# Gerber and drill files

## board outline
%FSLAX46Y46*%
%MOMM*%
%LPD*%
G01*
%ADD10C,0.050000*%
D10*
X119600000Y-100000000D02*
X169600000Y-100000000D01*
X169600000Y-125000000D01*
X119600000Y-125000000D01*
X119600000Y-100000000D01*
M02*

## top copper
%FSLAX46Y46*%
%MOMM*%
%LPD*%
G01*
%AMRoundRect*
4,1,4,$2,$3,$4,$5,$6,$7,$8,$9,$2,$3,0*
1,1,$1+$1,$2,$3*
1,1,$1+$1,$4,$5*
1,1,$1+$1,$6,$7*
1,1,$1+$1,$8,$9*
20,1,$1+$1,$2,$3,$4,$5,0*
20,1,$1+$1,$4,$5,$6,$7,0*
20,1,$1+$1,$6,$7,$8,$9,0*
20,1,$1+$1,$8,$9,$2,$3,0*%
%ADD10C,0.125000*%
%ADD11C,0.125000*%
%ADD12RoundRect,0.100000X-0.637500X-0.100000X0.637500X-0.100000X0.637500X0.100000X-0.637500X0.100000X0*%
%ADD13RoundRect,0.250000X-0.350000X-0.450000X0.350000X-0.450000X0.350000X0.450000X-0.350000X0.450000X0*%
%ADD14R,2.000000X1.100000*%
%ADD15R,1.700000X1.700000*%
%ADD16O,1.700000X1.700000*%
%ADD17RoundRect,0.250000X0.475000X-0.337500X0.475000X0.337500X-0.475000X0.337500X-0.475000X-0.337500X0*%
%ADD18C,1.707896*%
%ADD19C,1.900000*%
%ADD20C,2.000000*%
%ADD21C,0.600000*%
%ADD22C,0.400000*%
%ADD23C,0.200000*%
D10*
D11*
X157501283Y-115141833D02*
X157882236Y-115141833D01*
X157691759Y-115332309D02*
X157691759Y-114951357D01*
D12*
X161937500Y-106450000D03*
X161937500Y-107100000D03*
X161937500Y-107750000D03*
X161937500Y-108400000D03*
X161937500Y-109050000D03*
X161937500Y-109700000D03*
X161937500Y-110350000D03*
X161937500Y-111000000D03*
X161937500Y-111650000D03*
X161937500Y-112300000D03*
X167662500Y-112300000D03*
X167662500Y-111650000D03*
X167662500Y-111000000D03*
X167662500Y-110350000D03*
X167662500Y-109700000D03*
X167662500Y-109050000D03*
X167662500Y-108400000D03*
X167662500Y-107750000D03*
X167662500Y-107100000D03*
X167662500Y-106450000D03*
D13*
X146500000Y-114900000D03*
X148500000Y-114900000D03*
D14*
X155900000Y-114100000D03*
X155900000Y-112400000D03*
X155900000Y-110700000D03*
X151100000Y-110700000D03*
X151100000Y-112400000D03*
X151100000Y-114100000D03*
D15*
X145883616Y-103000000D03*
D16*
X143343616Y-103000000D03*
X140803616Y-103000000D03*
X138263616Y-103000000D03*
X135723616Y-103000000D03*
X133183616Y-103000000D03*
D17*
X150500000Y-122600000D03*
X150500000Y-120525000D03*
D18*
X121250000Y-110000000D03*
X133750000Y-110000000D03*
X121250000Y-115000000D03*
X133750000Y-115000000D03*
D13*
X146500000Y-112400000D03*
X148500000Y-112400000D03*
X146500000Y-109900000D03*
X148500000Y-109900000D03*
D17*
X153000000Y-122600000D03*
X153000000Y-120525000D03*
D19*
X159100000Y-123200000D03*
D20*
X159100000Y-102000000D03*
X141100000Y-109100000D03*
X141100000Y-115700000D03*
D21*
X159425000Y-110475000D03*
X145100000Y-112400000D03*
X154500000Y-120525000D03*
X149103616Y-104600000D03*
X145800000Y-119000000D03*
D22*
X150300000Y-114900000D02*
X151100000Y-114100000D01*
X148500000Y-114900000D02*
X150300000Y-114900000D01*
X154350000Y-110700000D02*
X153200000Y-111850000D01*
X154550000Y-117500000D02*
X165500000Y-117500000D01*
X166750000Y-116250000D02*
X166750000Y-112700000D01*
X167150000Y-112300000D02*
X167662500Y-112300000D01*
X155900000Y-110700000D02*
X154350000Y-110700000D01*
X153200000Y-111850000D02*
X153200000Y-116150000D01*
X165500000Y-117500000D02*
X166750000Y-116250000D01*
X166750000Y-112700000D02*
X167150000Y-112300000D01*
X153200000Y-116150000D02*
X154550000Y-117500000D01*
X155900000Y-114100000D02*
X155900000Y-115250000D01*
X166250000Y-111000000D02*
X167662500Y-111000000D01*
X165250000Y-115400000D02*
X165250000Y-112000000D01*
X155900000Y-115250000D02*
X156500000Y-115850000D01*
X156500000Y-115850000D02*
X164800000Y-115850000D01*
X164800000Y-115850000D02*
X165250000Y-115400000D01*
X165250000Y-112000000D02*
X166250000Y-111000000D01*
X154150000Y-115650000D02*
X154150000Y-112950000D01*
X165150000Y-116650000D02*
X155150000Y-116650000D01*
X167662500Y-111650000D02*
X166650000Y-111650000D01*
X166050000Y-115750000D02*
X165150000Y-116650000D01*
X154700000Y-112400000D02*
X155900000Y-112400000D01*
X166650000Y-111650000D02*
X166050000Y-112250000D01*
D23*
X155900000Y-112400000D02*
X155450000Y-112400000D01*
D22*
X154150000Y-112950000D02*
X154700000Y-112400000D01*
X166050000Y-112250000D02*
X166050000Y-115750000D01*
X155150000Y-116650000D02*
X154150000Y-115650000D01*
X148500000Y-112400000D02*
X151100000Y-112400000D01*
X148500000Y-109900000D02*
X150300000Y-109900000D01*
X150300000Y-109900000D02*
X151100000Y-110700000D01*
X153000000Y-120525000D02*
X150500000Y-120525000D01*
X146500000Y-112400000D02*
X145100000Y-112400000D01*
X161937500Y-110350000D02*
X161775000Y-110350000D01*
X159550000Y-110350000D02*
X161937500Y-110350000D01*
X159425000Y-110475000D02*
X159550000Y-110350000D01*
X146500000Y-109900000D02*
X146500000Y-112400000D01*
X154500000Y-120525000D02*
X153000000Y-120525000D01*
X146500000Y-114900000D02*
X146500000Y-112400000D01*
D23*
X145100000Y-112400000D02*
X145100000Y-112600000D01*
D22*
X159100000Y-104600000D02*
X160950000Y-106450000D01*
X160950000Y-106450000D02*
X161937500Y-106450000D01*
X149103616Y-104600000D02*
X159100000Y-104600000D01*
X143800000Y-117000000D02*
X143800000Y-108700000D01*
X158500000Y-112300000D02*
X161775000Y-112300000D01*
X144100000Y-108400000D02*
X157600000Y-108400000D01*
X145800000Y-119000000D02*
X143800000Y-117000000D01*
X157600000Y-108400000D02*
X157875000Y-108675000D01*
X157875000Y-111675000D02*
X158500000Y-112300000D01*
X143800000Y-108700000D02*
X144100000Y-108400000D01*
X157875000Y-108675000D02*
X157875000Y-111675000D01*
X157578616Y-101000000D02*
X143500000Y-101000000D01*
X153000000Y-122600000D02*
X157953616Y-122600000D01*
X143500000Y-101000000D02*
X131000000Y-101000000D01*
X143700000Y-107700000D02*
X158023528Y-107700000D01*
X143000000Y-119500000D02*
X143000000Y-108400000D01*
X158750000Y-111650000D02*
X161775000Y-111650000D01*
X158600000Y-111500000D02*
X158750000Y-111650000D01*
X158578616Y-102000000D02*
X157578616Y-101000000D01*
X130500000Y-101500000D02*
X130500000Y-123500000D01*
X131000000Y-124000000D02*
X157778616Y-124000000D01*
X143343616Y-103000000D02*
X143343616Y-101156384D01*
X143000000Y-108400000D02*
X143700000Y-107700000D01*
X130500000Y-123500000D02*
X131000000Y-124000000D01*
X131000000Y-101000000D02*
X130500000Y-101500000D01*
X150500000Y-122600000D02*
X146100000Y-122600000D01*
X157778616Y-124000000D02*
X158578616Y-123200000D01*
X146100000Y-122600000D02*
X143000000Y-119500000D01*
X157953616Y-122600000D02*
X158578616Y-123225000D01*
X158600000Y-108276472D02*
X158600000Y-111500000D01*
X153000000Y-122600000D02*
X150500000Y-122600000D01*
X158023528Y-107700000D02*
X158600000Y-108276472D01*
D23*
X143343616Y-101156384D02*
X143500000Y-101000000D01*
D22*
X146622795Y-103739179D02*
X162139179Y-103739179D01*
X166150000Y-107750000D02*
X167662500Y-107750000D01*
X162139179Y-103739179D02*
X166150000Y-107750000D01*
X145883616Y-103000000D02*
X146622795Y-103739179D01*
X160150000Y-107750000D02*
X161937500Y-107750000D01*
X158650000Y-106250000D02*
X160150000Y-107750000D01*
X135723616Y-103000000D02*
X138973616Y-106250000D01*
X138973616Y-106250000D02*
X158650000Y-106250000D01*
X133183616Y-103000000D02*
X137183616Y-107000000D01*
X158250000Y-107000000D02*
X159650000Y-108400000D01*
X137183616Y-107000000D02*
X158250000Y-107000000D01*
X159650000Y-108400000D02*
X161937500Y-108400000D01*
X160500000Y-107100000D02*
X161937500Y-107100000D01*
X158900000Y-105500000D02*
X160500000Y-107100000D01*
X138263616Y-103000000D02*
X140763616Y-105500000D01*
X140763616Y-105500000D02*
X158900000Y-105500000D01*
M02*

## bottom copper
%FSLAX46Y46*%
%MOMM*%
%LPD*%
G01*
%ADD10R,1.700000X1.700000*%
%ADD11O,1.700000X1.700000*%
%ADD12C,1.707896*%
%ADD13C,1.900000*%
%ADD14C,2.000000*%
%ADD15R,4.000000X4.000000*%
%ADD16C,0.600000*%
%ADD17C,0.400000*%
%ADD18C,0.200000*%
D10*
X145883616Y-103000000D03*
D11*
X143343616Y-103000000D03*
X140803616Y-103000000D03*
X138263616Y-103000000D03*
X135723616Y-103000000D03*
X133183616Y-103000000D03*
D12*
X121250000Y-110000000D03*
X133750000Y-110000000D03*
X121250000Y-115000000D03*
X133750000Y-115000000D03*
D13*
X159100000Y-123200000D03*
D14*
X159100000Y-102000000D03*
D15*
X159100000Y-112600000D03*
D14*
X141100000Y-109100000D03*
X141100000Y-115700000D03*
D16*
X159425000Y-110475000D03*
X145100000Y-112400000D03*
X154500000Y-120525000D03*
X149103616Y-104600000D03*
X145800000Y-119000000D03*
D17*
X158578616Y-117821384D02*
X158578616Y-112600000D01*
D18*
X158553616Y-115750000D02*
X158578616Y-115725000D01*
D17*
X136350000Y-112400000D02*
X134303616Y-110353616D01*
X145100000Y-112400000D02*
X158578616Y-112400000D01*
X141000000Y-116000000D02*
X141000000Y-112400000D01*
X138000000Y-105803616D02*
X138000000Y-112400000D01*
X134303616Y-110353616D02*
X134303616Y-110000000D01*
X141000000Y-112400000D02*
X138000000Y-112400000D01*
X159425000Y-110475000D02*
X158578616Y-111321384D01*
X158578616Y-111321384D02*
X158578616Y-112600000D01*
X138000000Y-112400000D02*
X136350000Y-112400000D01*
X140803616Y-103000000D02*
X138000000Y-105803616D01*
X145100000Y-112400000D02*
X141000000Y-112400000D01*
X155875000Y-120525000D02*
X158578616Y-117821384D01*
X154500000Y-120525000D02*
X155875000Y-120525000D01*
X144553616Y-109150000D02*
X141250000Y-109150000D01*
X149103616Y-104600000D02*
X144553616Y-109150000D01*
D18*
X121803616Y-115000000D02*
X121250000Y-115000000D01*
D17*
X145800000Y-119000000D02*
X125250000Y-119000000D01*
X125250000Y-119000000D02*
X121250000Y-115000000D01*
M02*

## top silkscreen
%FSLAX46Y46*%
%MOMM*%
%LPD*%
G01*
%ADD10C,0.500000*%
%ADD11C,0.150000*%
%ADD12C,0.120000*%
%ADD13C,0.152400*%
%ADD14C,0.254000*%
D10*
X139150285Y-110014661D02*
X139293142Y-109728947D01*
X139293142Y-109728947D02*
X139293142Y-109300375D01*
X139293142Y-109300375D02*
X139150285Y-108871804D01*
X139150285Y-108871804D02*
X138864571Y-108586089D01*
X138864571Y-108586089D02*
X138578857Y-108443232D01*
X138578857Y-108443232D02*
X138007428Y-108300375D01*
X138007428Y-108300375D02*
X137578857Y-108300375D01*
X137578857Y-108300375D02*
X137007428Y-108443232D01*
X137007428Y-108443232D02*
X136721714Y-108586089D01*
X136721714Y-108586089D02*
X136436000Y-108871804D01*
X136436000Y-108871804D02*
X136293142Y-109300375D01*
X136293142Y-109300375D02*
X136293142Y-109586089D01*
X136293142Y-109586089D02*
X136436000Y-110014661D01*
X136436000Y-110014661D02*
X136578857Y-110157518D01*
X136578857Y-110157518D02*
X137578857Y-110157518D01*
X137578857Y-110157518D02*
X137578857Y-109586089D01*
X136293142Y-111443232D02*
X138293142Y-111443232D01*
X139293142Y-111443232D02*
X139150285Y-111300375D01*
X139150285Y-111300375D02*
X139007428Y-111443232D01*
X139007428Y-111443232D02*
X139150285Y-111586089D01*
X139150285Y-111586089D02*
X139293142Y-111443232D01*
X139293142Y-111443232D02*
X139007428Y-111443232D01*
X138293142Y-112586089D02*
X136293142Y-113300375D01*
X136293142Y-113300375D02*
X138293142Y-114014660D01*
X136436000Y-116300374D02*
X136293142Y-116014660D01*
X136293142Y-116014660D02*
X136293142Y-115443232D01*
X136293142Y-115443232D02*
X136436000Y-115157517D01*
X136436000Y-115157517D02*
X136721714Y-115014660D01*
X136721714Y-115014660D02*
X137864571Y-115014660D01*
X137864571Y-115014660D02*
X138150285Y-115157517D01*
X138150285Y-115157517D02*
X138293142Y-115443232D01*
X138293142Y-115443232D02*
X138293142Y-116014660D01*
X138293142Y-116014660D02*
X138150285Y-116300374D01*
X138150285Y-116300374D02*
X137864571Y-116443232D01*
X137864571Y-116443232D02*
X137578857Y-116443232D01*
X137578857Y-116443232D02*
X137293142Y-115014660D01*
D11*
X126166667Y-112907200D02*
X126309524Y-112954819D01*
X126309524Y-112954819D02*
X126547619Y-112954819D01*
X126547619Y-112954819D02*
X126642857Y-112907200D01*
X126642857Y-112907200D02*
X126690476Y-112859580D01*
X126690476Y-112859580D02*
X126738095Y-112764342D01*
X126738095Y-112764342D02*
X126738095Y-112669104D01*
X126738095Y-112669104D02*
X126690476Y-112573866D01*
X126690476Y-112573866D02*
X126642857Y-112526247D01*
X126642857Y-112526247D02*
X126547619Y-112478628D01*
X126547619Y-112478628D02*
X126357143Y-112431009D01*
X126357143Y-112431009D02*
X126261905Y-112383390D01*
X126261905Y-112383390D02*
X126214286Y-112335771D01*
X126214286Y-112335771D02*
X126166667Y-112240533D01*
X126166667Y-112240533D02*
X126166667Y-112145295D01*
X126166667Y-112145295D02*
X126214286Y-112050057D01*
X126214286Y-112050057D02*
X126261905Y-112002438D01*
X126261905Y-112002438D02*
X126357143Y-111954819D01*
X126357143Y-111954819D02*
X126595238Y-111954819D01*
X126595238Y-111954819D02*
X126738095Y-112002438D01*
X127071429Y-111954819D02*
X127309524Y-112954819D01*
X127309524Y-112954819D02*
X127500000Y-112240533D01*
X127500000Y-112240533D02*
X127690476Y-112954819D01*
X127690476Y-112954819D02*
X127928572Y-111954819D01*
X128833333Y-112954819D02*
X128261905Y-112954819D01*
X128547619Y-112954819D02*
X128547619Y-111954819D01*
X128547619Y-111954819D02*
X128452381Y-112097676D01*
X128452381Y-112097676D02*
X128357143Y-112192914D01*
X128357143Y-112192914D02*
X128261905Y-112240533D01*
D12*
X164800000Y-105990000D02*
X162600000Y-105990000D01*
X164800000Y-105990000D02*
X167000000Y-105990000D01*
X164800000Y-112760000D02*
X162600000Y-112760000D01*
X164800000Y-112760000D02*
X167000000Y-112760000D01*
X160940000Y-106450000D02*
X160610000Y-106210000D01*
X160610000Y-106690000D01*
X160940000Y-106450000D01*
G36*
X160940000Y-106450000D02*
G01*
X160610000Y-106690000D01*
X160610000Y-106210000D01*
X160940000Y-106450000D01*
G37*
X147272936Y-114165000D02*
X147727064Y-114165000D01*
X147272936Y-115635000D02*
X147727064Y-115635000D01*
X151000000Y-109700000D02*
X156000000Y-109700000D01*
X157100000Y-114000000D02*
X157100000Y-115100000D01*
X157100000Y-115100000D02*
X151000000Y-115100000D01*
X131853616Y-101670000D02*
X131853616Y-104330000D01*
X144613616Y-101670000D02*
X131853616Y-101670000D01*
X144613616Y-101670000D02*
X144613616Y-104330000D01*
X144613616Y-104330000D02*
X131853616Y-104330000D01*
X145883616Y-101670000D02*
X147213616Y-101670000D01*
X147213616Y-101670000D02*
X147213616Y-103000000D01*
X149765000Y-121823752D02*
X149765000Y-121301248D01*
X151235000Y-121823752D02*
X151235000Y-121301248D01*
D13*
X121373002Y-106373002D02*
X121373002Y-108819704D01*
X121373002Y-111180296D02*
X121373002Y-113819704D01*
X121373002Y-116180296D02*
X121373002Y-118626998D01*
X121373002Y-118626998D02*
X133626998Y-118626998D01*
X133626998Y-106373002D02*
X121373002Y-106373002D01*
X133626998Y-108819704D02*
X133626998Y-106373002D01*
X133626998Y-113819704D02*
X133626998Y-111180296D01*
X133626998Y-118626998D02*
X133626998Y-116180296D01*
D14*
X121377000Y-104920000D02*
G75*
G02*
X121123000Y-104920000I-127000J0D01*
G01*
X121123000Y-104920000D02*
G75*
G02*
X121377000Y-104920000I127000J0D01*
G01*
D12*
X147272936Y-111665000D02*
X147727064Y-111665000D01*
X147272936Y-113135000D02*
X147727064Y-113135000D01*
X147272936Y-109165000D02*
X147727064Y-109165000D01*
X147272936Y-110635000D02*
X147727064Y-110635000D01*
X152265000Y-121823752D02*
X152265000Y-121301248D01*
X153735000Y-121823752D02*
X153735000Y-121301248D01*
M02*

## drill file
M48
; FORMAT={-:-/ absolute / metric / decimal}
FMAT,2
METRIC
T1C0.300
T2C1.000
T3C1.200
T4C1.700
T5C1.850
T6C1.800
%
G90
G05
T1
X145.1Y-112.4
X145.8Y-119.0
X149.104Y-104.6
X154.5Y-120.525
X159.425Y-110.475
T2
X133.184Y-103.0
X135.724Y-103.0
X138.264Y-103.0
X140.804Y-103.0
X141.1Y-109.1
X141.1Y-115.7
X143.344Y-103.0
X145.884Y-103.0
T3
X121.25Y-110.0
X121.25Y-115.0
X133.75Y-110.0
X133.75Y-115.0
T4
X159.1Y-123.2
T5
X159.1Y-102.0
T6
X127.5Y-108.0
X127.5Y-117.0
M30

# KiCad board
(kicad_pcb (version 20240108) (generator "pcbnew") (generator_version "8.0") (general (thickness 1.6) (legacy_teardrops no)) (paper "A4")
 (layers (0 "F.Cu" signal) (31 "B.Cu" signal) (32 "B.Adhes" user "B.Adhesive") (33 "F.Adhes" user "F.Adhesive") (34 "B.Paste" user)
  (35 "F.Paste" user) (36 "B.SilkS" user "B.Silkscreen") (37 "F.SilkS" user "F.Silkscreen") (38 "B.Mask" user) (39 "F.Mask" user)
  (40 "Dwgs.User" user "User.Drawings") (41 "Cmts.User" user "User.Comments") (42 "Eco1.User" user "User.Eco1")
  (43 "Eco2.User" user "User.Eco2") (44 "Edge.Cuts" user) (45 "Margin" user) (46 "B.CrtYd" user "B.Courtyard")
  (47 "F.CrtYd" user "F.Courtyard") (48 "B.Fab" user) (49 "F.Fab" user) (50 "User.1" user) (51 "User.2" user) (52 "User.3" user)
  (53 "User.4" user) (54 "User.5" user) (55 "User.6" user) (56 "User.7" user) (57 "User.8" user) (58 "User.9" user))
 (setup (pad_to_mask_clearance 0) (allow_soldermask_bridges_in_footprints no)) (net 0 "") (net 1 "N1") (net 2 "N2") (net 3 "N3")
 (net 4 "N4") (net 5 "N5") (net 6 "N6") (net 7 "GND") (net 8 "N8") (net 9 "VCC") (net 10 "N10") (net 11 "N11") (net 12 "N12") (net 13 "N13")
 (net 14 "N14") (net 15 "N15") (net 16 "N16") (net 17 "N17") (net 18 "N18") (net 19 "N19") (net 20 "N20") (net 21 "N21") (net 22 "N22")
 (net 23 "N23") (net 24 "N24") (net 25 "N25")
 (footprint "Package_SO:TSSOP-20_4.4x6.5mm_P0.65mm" (layer "F.Cu") (at 164.8 109.375)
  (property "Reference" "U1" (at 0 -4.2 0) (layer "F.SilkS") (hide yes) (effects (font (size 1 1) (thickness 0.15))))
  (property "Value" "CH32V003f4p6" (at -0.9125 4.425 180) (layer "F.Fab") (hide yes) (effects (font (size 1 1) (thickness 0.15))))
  (fp_line (start 0 -3.385) (end -2.2 -3.385) (stroke (width 0.12) (type solid)) (layer "F.SilkS"))
  (fp_line (start 0 -3.385) (end 2.2 -3.385) (stroke (width 0.12) (type solid)) (layer "F.SilkS"))
  (fp_line (start 0 3.385) (end -2.2 3.385) (stroke (width 0.12) (type solid)) (layer "F.SilkS"))
  (fp_line (start 0 3.385) (end 2.2 3.385) (stroke (width 0.12) (type solid)) (layer "F.SilkS"))
  (fp_poly
   (pts (xy -3.86 -2.925) (xy -4.19 -3.165) (xy -4.19 -2.685) (xy -3.86 -2.925)) (stroke (width 0.12) (type solid)) (fill solid)
   (layer "F.SilkS"))
  (pad "1" smd roundrect (at -2.8625 -2.925) (size 1.475 0.4) (layers "F.Cu" "F.Paste" "F.Mask") (roundrect_rratio 0.25) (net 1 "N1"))
  (pad "2" smd roundrect (at -2.8625 -2.275) (size 1.475 0.4) (layers "F.Cu" "F.Paste" "F.Mask") (roundrect_rratio 0.25) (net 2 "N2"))
  (pad "3" smd roundrect (at -2.8625 -1.625) (size 1.475 0.4) (layers "F.Cu" "F.Paste" "F.Mask") (roundrect_rratio 0.25) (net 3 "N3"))
  (pad "4" smd roundrect (at -2.8625 -0.975) (size 1.475 0.4) (layers "F.Cu" "F.Paste" "F.Mask") (roundrect_rratio 0.25) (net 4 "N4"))
  (pad "5" smd roundrect (at -2.8625 -0.325) (size 1.475 0.4) (layers "F.Cu" "F.Paste" "F.Mask") (roundrect_rratio 0.25) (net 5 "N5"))
  (pad "6" smd roundrect (at -2.8625 0.325) (size 1.475 0.4) (layers "F.Cu" "F.Paste" "F.Mask") (roundrect_rratio 0.25) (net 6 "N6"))
  (pad "7" smd roundrect (at -2.8625 0.975) (size 1.475 0.4) (layers "F.Cu" "F.Paste" "F.Mask") (roundrect_rratio 0.25) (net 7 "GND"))
  (pad "8" smd roundrect (at -2.8625 1.625) (size 1.475 0.4) (layers "F.Cu" "F.Paste" "F.Mask") (roundrect_rratio 0.25) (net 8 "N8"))
  (pad "9" smd roundrect (at -2.8625 2.275) (size 1.475 0.4) (layers "F.Cu" "F.Paste" "F.Mask") (roundrect_rratio 0.25) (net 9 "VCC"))
  (pad "10" smd roundrect (at -2.8625 2.925) (size 1.475 0.4) (layers "F.Cu" "F.Paste" "F.Mask") (roundrect_rratio 0.25) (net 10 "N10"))
  (pad "11" smd roundrect (at 2.8625 2.925) (size 1.475 0.4) (layers "F.Cu" "F.Paste" "F.Mask") (roundrect_rratio 0.25) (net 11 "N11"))
  (pad "12" smd roundrect (at 2.8625 2.275) (size 1.475 0.4) (layers "F.Cu" "F.Paste" "F.Mask") (roundrect_rratio 0.25) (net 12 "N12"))
  (pad "13" smd roundrect (at 2.8625 1.625) (size 1.475 0.4) (layers "F.Cu" "F.Paste" "F.Mask") (roundrect_rratio 0.25) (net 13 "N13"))
  (pad "14" smd roundrect (at 2.8625 0.975) (size 1.475 0.4) (layers "F.Cu" "F.Paste" "F.Mask") (roundrect_rratio 0.25) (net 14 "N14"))
  (pad "15" smd roundrect (at 2.8625 0.325) (size 1.475 0.4) (layers "F.Cu" "F.Paste" "F.Mask") (roundrect_rratio 0.25) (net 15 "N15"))
  (pad "16" smd roundrect (at 2.8625 -0.325) (size 1.475 0.4) (layers "F.Cu" "F.Paste" "F.Mask") (roundrect_rratio 0.25) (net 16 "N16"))
  (pad "17" smd roundrect (at 2.8625 -0.975) (size 1.475 0.4) (layers "F.Cu" "F.Paste" "F.Mask") (roundrect_rratio 0.25) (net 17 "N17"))
  (pad "18" smd roundrect (at 2.8625 -1.625) (size 1.475 0.4) (layers "F.Cu" "F.Paste" "F.Mask") (roundrect_rratio 0.25) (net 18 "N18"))
  (pad "19" smd roundrect (at 2.8625 -2.275) (size 1.475 0.4) (layers "F.Cu" "F.Paste" "F.Mask") (roundrect_rratio 0.25) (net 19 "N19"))
  (pad "20" smd roundrect (at 2.8625 -2.925) (size 1.475 0.4) (layers "F.Cu" "F.Paste" "F.Mask") (roundrect_rratio 0.25) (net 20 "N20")))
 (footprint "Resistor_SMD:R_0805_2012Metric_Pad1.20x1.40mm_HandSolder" (layer "F.Cu") (at 147.5 114.9)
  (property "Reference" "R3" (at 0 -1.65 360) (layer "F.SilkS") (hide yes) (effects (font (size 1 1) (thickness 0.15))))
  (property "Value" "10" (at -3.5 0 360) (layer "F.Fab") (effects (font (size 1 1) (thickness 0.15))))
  (fp_line (start -0.227064 -0.735) (end 0.227064 -0.735) (stroke (width 0.12) (type solid)) (layer "F.SilkS"))
  (fp_line (start -0.227064 0.735) (end 0.227064 0.735) (stroke (width 0.12) (type solid)) (layer "F.SilkS"))
  (pad "1" smd roundrect (at -1 0) (size 1.2 1.4) (layers "F.Cu" "F.Paste" "F.Mask") (roundrect_rratio 0.208333) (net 7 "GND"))
  (pad "2" smd roundrect (at 1 0) (size 1.2 1.4) (layers "F.Cu" "F.Paste" "F.Mask") (roundrect_rratio 0.208333) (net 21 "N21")))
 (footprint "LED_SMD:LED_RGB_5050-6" (layer "F.Cu") (at 153.5 112.4 180)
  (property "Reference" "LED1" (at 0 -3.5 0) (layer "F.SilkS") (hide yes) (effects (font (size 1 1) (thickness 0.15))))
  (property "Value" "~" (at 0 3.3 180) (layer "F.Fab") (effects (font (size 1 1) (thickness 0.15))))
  (fp_line (start 2.5 2.7) (end -2.5 2.7) (stroke (width 0.12) (type solid)) (layer "F.SilkS"))
  (fp_line (start -3.6 -1.6) (end -3.6 -2.7) (stroke (width 0.12) (type solid)) (layer "F.SilkS"))
  (fp_line (start -3.6 -2.7) (end 2.5 -2.7) (stroke (width 0.12) (type solid)) (layer "F.SilkS"))
  (pad "1" smd rect (at -2.4 -1.7 270) (size 1.1 2) (layers "F.Cu" "F.Paste" "F.Mask") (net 13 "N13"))
  (pad "2" smd rect (at -2.4 0 270) (size 1.1 2) (layers "F.Cu" "F.Paste" "F.Mask") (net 12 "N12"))
  (pad "3" smd rect (at -2.4 1.7 270) (size 1.1 2) (layers "F.Cu" "F.Paste" "F.Mask") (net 11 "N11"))
  (pad "4" smd rect (at 2.4 1.7 270) (size 1.1 2) (layers "F.Cu" "F.Paste" "F.Mask") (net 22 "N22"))
  (pad "5" smd rect (at 2.4 0 270) (size 1.1 2) (layers "F.Cu" "F.Paste" "F.Mask") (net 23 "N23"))
  (pad "6" smd rect (at 2.4 -1.7 270) (size 1.1 2) (layers "F.Cu" "F.Paste" "F.Mask") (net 21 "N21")))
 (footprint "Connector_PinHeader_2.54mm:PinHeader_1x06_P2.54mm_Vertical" (layer "F.Cu") (at 145.883616 103 -90)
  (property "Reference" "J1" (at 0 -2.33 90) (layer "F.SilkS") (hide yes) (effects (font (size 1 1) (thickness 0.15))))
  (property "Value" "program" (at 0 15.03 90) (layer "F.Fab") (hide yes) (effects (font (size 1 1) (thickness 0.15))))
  (fp_line (start -1.33 14.03) (end 1.33 14.03) (stroke (width 0.12) (type solid)) (layer "F.SilkS"))
  (fp_line (start -1.33 1.27) (end -1.33 14.03) (stroke (width 0.12) (type solid)) (layer "F.SilkS"))
  (fp_line (start -1.33 1.27) (end 1.33 1.27) (stroke (width 0.12) (type solid)) (layer "F.SilkS"))
  (fp_line (start 1.33 1.27) (end 1.33 14.03) (stroke (width 0.12) (type solid)) (layer "F.SilkS"))
  (fp_line (start -1.33 0) (end -1.33 -1.33) (stroke (width 0.12) (type solid)) (layer "F.SilkS"))
  (fp_line (start -1.33 -1.33) (end 0 -1.33) (stroke (width 0.12) (type solid)) (layer "F.SilkS"))
  (pad "1" thru_hole rect (at 0 0 270) (size 1.7 1.7) (drill 1) (layers "*.Cu" "*.Mask") (remove_unused_layers no) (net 18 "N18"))
  (pad "2" thru_hole oval (at 0 2.54 270) (size 1.7 1.7) (drill 1) (layers "*.Cu" "*.Mask") (remove_unused_layers no) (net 9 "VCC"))
  (pad "3" thru_hole oval (at 0 5.08 270) (size 1.7 1.7) (drill 1) (layers "*.Cu" "*.Mask") (remove_unused_layers no) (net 7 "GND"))
  (pad "4" thru_hole oval (at 0 7.62 270) (size 1.7 1.7) (drill 1) (layers "*.Cu" "*.Mask") (remove_unused_layers no) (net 2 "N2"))
  (pad "5" thru_hole oval (at 0 10.16 270) (size 1.7 1.7) (drill 1) (layers "*.Cu" "*.Mask") (remove_unused_layers no) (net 3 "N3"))
  (pad "6" thru_hole oval (at 0 12.7 270) (size 1.7 1.7) (drill 1) (layers "*.Cu" "*.Mask") (remove_unused_layers no) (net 4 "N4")))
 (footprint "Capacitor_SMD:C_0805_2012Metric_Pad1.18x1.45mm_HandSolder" (layer "F.Cu") (at 150.5 121.5625 90)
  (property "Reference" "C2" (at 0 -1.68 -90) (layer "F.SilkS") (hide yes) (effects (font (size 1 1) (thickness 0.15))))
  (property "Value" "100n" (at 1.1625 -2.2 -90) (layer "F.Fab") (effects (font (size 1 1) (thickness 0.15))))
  (fp_line (start -0.261252 -0.735) (end 0.261252 -0.735) (stroke (width 0.12) (type solid)) (layer "F.SilkS"))
  (fp_line (start -0.261252 0.735) (end 0.261252 0.735) (stroke (width 0.12) (type solid)) (layer "F.SilkS"))
  (pad "1" smd roundrect (at -1.0375 0 90) (size 1.175 1.45) (layers "F.Cu" "F.Paste" "F.Mask") (roundrect_rratio 0.212766) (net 9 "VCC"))
  (pad "2" smd roundrect (at 1.0375 0 90) (size 1.175 1.45) (layers "F.Cu" "F.Paste" "F.Mask") (roundrect_rratio 0.212766) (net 7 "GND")))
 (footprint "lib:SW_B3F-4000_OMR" (layer "F.Cu") (at 121.25 110)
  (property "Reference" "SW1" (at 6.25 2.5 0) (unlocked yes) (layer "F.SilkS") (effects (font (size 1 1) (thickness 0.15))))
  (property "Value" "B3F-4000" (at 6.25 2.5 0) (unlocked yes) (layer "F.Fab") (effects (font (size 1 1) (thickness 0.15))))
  (fp_line (start 0.123002 -3.626998) (end 0.123002 -1.180296) (stroke (width 0.1524) (type solid)) (layer "F.SilkS"))
  (fp_line (start 0.123002 1.180296) (end 0.123002 3.819704) (stroke (width 0.1524) (type solid)) (layer "F.SilkS"))
  (fp_line (start 0.123002 6.180296) (end 0.123002 8.626998) (stroke (width 0.1524) (type solid)) (layer "F.SilkS"))
  (fp_line (start 0.123002 8.626998) (end 12.376998 8.626998) (stroke (width 0.1524) (type solid)) (layer "F.SilkS"))
  (fp_line (start 12.376998 -3.626998) (end 0.123002 -3.626998) (stroke (width 0.1524) (type solid)) (layer "F.SilkS"))
  (fp_line (start 12.376998 -1.180296) (end 12.376998 -3.626998) (stroke (width 0.1524) (type solid)) (layer "F.SilkS"))
  (fp_line (start 12.376998 3.819704) (end 12.376998 1.180296) (stroke (width 0.1524) (type solid)) (layer "F.SilkS"))
  (fp_line (start 12.376998 8.626998) (end 12.376998 6.180296) (stroke (width 0.1524) (type solid)) (layer "F.SilkS"))
  (fp_circle (center 0 -5.08) (end 0.127 -5.08) (stroke (width 0.254) (type solid)) (fill none) (layer "F.SilkS"))
  (pad "" np_thru_hole circle (at 6.25 -2) (size 1.799996 1.799996) (drill 1.799996) (layers "*.Cu" "*.Mask"))
  (pad "" np_thru_hole circle (at 6.25 7) (size 1.799996 1.799996) (drill 1.799996) (layers "*.Cu" "*.Mask"))
  (pad "1" thru_hole circle (at 0 0) (size 1.707896 1.707896) (drill 1.199896) (layers "*.Cu" "*.Mask") (remove_unused_layers no)
   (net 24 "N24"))
  (pad "2" thru_hole circle (at 12.5 0) (size 1.707896 1.707896) (drill 1.199896) (layers "*.Cu" "*.Mask") (remove_unused_layers no)
   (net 7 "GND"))
  (pad "3" thru_hole circle (at 0 5) (size 1.707896 1.707896) (drill 1.199896) (layers "*.Cu" "*.Mask") (remove_unused_layers no)
   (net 10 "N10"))
  (pad "4" thru_hole circle (at 12.5 5) (size 1.707896 1.707896) (drill 1.199896) (layers "*.Cu" "*.Mask") (remove_unused_layers no)
   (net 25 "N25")))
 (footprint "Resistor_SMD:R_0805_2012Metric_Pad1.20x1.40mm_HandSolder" (layer "F.Cu") (at 147.5 112.4)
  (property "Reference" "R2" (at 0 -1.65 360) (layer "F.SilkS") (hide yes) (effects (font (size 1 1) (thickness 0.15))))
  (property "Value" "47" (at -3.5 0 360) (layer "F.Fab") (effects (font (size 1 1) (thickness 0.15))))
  (fp_line (start -0.227064 -0.735) (end 0.227064 -0.735) (stroke (width 0.12) (type solid)) (layer "F.SilkS"))
  (fp_line (start -0.227064 0.735) (end 0.227064 0.735) (stroke (width 0.12) (type solid)) (layer "F.SilkS"))
  (pad "1" smd roundrect (at -1 0) (size 1.2 1.4) (layers "F.Cu" "F.Paste" "F.Mask") (roundrect_rratio 0.208333) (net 7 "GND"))
  (pad "2" smd roundrect (at 1 0) (size 1.2 1.4) (layers "F.Cu" "F.Paste" "F.Mask") (roundrect_rratio 0.208333) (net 23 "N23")))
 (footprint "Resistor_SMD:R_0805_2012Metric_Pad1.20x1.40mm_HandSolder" (layer "F.Cu") (at 147.5 109.9)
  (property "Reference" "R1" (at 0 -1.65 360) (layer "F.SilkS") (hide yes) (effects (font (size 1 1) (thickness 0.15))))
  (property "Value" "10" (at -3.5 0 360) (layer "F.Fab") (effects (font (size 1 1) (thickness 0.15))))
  (fp_line (start -0.227064 -0.735) (end 0.227064 -0.735) (stroke (width 0.12) (type solid)) (layer "F.SilkS"))
  (fp_line (start -0.227064 0.735) (end 0.227064 0.735) (stroke (width 0.12) (type solid)) (layer "F.SilkS"))
  (pad "1" smd roundrect (at -1 0) (size 1.2 1.4) (layers "F.Cu" "F.Paste" "F.Mask") (roundrect_rratio 0.208333) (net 7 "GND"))
  (pad "2" smd roundrect (at 1 0) (size 1.2 1.4) (layers "F.Cu" "F.Paste" "F.Mask") (roundrect_rratio 0.208333) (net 22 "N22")))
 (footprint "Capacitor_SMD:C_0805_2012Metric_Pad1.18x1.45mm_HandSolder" (layer "F.Cu") (at 153 121.5625 90)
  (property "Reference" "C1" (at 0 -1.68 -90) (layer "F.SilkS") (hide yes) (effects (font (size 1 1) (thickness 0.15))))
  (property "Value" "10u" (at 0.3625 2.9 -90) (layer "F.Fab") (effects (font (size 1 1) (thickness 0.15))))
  (fp_line (start -0.261252 -0.735) (end 0.261252 -0.735) (stroke (width 0.12) (type solid)) (layer "F.SilkS"))
  (fp_line (start -0.261252 0.735) (end 0.261252 0.735) (stroke (width 0.12) (type solid)) (layer "F.SilkS"))
  (pad "1" smd roundrect (at -1.0375 0 90) (size 1.175 1.45) (layers "F.Cu" "F.Paste" "F.Mask") (roundrect_rratio 0.212766) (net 9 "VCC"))
  (pad "2" smd roundrect (at 1.0375 0 90) (size 1.175 1.45) (layers "F.Cu" "F.Paste" "F.Mask") (roundrect_rratio 0.212766) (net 7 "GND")))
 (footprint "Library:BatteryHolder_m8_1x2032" (layer "B.Cu") (at 159.1 112.6 90)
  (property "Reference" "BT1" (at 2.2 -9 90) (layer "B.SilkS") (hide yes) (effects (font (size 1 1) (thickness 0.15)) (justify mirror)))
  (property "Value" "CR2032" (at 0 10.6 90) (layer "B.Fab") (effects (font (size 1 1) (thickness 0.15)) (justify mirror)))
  (pad "1" thru_hole circle (at -10.6 0 90) (size 1.9 1.9) (drill 1.7) (layers "*.Cu" "*.Mask") (remove_unused_layers no) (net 9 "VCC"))
  (pad "1" thru_hole circle (at 10.6 0 90) (size 2 2) (drill 1.85) (layers "*.Cu" "*.Mask") (remove_unused_layers no) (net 9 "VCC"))
  (pad "2" smd rect (at 0 0 90) (size 4 4) (layers "B.Cu" "B.Paste" "B.Mask") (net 7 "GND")))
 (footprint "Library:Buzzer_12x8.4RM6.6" (layer "B.Cu") (at 141.1 109.1 -90)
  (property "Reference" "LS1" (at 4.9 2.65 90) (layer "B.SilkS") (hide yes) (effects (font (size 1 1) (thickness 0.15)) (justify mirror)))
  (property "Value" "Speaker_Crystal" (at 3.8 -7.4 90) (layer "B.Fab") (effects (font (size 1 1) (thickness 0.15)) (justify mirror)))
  (pad "1" thru_hole circle (at 0 0 270) (size 2 2) (drill 1) (layers "*.Cu" "*.Mask") (remove_unused_layers no) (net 1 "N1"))
  (pad "2" thru_hole circle (at 6.6 0 270) (size 2 2) (drill 1) (layers "*.Cu" "*.Mask") (remove_unused_layers no) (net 7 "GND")))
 (gr_rect (start 119.6 100) (end 169.6 125) (stroke (width 0.05) (type default)) (fill none) (layer "Edge.Cuts"))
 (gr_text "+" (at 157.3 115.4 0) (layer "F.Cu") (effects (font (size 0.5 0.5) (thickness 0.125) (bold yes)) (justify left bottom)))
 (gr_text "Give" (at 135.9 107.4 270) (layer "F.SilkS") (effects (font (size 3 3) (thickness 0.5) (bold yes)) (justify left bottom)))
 (segment (start 150.3 114.9) (end 151.1 114.1) (width 0.4) (layer "F.Cu") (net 21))
 (segment (start 148.5 114.9) (end 150.3 114.9) (width 0.4) (layer "F.Cu") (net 21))
 (segment (start 154.35 110.7) (end 153.2 111.85) (width 0.4) (layer "F.Cu") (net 11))
 (segment (start 154.55 117.5) (end 165.5 117.5) (width 0.4) (layer "F.Cu") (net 11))
 (segment (start 166.75 116.25) (end 166.75 112.7) (width 0.4) (layer "F.Cu") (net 11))
 (segment (start 167.15 112.3) (end 167.6625 112.3) (width 0.4) (layer "F.Cu") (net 11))
 (segment (start 155.9 110.7) (end 154.35 110.7) (width 0.4) (layer "F.Cu") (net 11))
 (segment (start 153.2 111.85) (end 153.2 116.15) (width 0.4) (layer "F.Cu") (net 11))
 (segment (start 165.5 117.5) (end 166.75 116.25) (width 0.4) (layer "F.Cu") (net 11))
 (segment (start 166.75 112.7) (end 167.15 112.3) (width 0.4) (layer "F.Cu") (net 11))
 (segment (start 153.2 116.15) (end 154.55 117.5) (width 0.4) (layer "F.Cu") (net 11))
 (segment (start 155.9 114.1) (end 155.9 115.25) (width 0.4) (layer "F.Cu") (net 13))
 (segment (start 166.25 111) (end 167.6625 111) (width 0.4) (layer "F.Cu") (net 13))
 (segment (start 165.25 115.4) (end 165.25 112) (width 0.4) (layer "F.Cu") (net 13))
 (segment (start 155.9 115.25) (end 156.5 115.85) (width 0.4) (layer "F.Cu") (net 13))
 (segment (start 156.5 115.85) (end 164.8 115.85) (width 0.4) (layer "F.Cu") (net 13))
 (segment (start 164.8 115.85) (end 165.25 115.4) (width 0.4) (layer "F.Cu") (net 13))
 (segment (start 165.25 112) (end 166.25 111) (width 0.4) (layer "F.Cu") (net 13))
 (segment (start 154.15 115.65) (end 154.15 112.95) (width 0.4) (layer "F.Cu") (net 12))
 (segment (start 165.15 116.65) (end 155.15 116.65) (width 0.4) (layer "F.Cu") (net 12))
 (segment (start 167.6625 111.65) (end 166.65 111.65) (width 0.4) (layer "F.Cu") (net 12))
 (segment (start 166.05 115.75) (end 165.15 116.65) (width 0.4) (layer "F.Cu") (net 12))
 (segment (start 154.7 112.4) (end 155.9 112.4) (width 0.4) (layer "F.Cu") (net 12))
 (segment (start 166.65 111.65) (end 166.05 112.25) (width 0.4) (layer "F.Cu") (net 12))
 (segment (start 155.9 112.4) (end 155.45 112.4) (width 0.2) (layer "F.Cu") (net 12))
 (segment (start 154.15 112.95) (end 154.7 112.4) (width 0.4) (layer "F.Cu") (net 12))
 (segment (start 166.05 112.25) (end 166.05 115.75) (width 0.4) (layer "F.Cu") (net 12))
 (segment (start 155.15 116.65) (end 154.15 115.65) (width 0.4) (layer "F.Cu") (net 12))
 (segment (start 148.5 112.4) (end 151.1 112.4) (width 0.4) (layer "F.Cu") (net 23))
 (segment (start 148.5 109.9) (end 150.3 109.9) (width 0.4) (layer "F.Cu") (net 22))
 (segment (start 150.3 109.9) (end 151.1 110.7) (width 0.4) (layer "F.Cu") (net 22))
 (segment (start 153 120.525) (end 150.5 120.525) (width 0.4) (layer "F.Cu") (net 7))
 (segment (start 146.5 112.4) (end 145.1 112.4) (width 0.4) (layer "F.Cu") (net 7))
 (segment (start 161.9375 110.35) (end 161.775 110.35) (width 0.4) (layer "F.Cu") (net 7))
 (segment (start 159.55 110.35) (end 161.9375 110.35) (width 0.4) (layer "F.Cu") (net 7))
 (segment (start 159.425 110.475) (end 159.55 110.35) (width 0.4) (layer "F.Cu") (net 7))
 (segment (start 146.5 109.9) (end 146.5 112.4) (width 0.4) (layer "F.Cu") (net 7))
 (segment (start 154.5 120.525) (end 153 120.525) (width 0.4) (layer "F.Cu") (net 7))
 (segment (start 146.5 114.9) (end 146.5 112.4) (width 0.4) (layer "F.Cu") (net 7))
 (segment (start 145.1 112.4) (end 145.1 112.6) (width 0.2) (layer "F.Cu") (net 7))
 (via (at 159.425 110.475) (size 0.6) (drill 0.3) (layers "F.Cu" "B.Cu") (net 7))
 (via (at 145.1 112.4) (size 0.6) (drill 0.3) (layers "F.Cu" "B.Cu") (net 7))
 (via (at 154.5 120.525) (size 0.6) (drill 0.3) (layers "F.Cu" "B.Cu") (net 7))
 (segment (start 158.578616 117.821384) (end 158.578616 112.6) (width 0.4) (layer "B.Cu") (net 7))
 (segment (start 158.553616 115.75) (end 158.578616 115.725) (width 0.2) (layer "B.Cu") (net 7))
 (segment (start 136.35 112.4) (end 134.303616 110.353616) (width 0.4) (layer "B.Cu") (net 7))
 (segment (start 145.1 112.4) (end 158.578616 112.4) (width 0.4) (layer "B.Cu") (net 7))
 (segment (start 141 116) (end 141 112.4) (width 0.4) (layer "B.Cu") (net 7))
 (segment (start 138 105.803616) (end 138 112.4) (width 0.4) (layer "B.Cu") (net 7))
 (segment (start 134.303616 110.353616) (end 134.303616 110) (width 0.4) (layer "B.Cu") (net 7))
 (segment (start 141 112.4) (end 138 112.4) (width 0.4) (layer "B.Cu") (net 7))
 (segment (start 159.425 110.475) (end 158.578616 111.321384) (width 0.4) (layer "B.Cu") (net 7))
 (segment (start 158.578616 111.321384) (end 158.578616 112.6) (width 0.4) (layer "B.Cu") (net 7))
 (segment (start 138 112.4) (end 136.35 112.4) (width 0.4) (layer "B.Cu") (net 7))
 (segment (start 140.803616 103) (end 138 105.803616) (width 0.4) (layer "B.Cu") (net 7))
 (segment (start 145.1 112.4) (end 141 112.4) (width 0.4) (layer "B.Cu") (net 7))
 (segment (start 155.875 120.525) (end 158.578616 117.821384) (width 0.4) (layer "B.Cu") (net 7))
 (segment (start 154.5 120.525) (end 155.875 120.525) (width 0.4) (layer "B.Cu") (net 7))
 (segment (start 159.1 104.6) (end 160.95 106.45) (width 0.4) (layer "F.Cu") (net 1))
 (segment (start 160.95 106.45) (end 161.9375 106.45) (width 0.4) (layer "F.Cu") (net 1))
 (segment (start 149.103616 104.6) (end 159.1 104.6) (width 0.4) (layer "F.Cu") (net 1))
 (via (at 149.103616 104.6) (size 0.6) (drill 0.3) (layers "F.Cu" "B.Cu") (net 1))
 (segment (start 144.553616 109.15) (end 141.25 109.15) (width 0.4) (layer "B.Cu") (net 1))
 (segment (start 149.103616 104.6) (end 144.553616 109.15) (width 0.4) (layer "B.Cu") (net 1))
 (segment (start 143.8 117) (end 143.8 108.7) (width 0.4) (layer "F.Cu") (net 10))
 (segment (start 158.5 112.3) (end 161.775 112.3) (width 0.4) (layer "F.Cu") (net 10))
 (segment (start 144.1 108.4) (end 157.6 108.4) (width 0.4) (layer "F.Cu") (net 10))
 (segment (start 145.8 119) (end 143.8 117) (width 0.4) (layer "F.Cu") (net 10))
 (segment (start 157.6 108.4) (end 157.875 108.675) (width 0.4) (layer "F.Cu") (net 10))
 (segment (start 157.875 111.675) (end 158.5 112.3) (width 0.4) (layer "F.Cu") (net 10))
 (segment (start 143.8 108.7) (end 144.1 108.4) (width 0.4) (layer "F.Cu") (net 10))
 (segment (start 157.875 108.675) (end 157.875 111.675) (width 0.4) (layer "F.Cu") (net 10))
 (via (at 145.8 119) (size 0.6) (drill 0.3) (layers "F.Cu" "B.Cu") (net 10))
 (segment (start 121.803616 115) (end 121.25 115) (width 0.2) (layer "B.Cu") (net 10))
 (segment (start 145.8 119) (end 125.25 119) (width 0.4) (layer "B.Cu") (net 10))
 (segment (start 125.25 119) (end 121.25 115) (width 0.4) (layer "B.Cu") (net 10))
 (segment (start 157.578616 101) (end 143.5 101) (width 0.4) (layer "F.Cu") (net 9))
 (segment (start 153 122.6) (end 157.953616 122.6) (width 0.4) (layer "F.Cu") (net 9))
 (segment (start 143.5 101) (end 131 101) (width 0.4) (layer "F.Cu") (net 9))
 (segment (start 143.7 107.7) (end 158.023528 107.7) (width 0.4) (layer "F.Cu") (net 9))
 (segment (start 143 119.5) (end 143 108.4) (width 0.4) (layer "F.Cu") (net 9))
 (segment (start 158.75 111.65) (end 161.775 111.65) (width 0.4) (layer "F.Cu") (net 9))
 (segment (start 158.6 111.5) (end 158.75 111.65) (width 0.4) (layer "F.Cu") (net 9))
 (segment (start 158.578616 102) (end 157.578616 101) (width 0.4) (layer "F.Cu") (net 9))
 (segment (start 130.5 101.5) (end 130.5 123.5) (width 0.4) (layer "F.Cu") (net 9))
 (segment (start 131 124) (end 157.778616 124) (width 0.4) (layer "F.Cu") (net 9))
 (segment (start 143.343616 103) (end 143.343616 101.156384) (width 0.4) (layer "F.Cu") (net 9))
 (segment (start 143 108.4) (end 143.7 107.7) (width 0.4) (layer "F.Cu") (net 9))
 (segment (start 130.5 123.5) (end 131 124) (width 0.4) (layer "F.Cu") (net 9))
 (segment (start 131 101) (end 130.5 101.5) (width 0.4) (layer "F.Cu") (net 9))
 (segment (start 150.5 122.6) (end 146.1 122.6) (width 0.4) (layer "F.Cu") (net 9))
 (segment (start 157.778616 124) (end 158.578616 123.2) (width 0.4) (layer "F.Cu") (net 9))
 (segment (start 146.1 122.6) (end 143 119.5) (width 0.4) (layer "F.Cu") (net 9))
 (segment (start 157.953616 122.6) (end 158.578616 123.225) (width 0.4) (layer "F.Cu") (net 9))
 (segment (start 158.6 108.276472) (end 158.6 111.5) (width 0.4) (layer "F.Cu") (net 9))
 (segment (start 153 122.6) (end 150.5 122.6) (width 0.4) (layer "F.Cu") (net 9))
 (segment (start 158.023528 107.7) (end 158.6 108.276472) (width 0.4) (layer "F.Cu") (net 9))
 (segment (start 143.343616 101.156384) (end 143.5 101) (width 0.2) (layer "F.Cu") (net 9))
 (segment (start 146.622795 103.739179) (end 162.139179 103.739179) (width 0.4) (layer "F.Cu") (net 18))
 (segment (start 166.15 107.75) (end 167.6625 107.75) (width 0.4) (layer "F.Cu") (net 18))
 (segment (start 162.139179 103.739179) (end 166.15 107.75) (width 0.4) (layer "F.Cu") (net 18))
 (segment (start 145.883616 103) (end 146.622795 103.739179) (width 0.4) (layer "F.Cu") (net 18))
 (segment (start 160.15 107.75) (end 161.9375 107.75) (width 0.4) (layer "F.Cu") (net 3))
 (segment (start 158.65 106.25) (end 160.15 107.75) (width 0.4) (layer "F.Cu") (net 3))
 (segment (start 135.723616 103) (end 138.973616 106.25) (width 0.4) (layer "F.Cu") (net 3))
 (segment (start 138.973616 106.25) (end 158.65 106.25) (width 0.4) (layer "F.Cu") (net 3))
 (segment (start 133.183616 103) (end 137.183616 107) (width 0.4) (layer "F.Cu") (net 4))
 (segment (start 158.25 107) (end 159.65 108.4) (width 0.4) (layer "F.Cu") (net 4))
 (segment (start 137.183616 107) (end 158.25 107) (width 0.4) (layer "F.Cu") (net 4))
 (segment (start 159.65 108.4) (end 161.9375 108.4) (width 0.4) (layer "F.Cu") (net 4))
 (segment (start 160.5 107.1) (end 161.9375 107.1) (width 0.4) (layer "F.Cu") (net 2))
 (segment (start 158.9 105.5) (end 160.5 107.1) (width 0.4) (layer "F.Cu") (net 2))
 (segment (start 138.263616 103) (end 140.763616 105.5) (width 0.4) (layer "F.Cu") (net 2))
 (segment (start 140.763616 105.5) (end 158.9 105.5) (width 0.4) (layer "F.Cu") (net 2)))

